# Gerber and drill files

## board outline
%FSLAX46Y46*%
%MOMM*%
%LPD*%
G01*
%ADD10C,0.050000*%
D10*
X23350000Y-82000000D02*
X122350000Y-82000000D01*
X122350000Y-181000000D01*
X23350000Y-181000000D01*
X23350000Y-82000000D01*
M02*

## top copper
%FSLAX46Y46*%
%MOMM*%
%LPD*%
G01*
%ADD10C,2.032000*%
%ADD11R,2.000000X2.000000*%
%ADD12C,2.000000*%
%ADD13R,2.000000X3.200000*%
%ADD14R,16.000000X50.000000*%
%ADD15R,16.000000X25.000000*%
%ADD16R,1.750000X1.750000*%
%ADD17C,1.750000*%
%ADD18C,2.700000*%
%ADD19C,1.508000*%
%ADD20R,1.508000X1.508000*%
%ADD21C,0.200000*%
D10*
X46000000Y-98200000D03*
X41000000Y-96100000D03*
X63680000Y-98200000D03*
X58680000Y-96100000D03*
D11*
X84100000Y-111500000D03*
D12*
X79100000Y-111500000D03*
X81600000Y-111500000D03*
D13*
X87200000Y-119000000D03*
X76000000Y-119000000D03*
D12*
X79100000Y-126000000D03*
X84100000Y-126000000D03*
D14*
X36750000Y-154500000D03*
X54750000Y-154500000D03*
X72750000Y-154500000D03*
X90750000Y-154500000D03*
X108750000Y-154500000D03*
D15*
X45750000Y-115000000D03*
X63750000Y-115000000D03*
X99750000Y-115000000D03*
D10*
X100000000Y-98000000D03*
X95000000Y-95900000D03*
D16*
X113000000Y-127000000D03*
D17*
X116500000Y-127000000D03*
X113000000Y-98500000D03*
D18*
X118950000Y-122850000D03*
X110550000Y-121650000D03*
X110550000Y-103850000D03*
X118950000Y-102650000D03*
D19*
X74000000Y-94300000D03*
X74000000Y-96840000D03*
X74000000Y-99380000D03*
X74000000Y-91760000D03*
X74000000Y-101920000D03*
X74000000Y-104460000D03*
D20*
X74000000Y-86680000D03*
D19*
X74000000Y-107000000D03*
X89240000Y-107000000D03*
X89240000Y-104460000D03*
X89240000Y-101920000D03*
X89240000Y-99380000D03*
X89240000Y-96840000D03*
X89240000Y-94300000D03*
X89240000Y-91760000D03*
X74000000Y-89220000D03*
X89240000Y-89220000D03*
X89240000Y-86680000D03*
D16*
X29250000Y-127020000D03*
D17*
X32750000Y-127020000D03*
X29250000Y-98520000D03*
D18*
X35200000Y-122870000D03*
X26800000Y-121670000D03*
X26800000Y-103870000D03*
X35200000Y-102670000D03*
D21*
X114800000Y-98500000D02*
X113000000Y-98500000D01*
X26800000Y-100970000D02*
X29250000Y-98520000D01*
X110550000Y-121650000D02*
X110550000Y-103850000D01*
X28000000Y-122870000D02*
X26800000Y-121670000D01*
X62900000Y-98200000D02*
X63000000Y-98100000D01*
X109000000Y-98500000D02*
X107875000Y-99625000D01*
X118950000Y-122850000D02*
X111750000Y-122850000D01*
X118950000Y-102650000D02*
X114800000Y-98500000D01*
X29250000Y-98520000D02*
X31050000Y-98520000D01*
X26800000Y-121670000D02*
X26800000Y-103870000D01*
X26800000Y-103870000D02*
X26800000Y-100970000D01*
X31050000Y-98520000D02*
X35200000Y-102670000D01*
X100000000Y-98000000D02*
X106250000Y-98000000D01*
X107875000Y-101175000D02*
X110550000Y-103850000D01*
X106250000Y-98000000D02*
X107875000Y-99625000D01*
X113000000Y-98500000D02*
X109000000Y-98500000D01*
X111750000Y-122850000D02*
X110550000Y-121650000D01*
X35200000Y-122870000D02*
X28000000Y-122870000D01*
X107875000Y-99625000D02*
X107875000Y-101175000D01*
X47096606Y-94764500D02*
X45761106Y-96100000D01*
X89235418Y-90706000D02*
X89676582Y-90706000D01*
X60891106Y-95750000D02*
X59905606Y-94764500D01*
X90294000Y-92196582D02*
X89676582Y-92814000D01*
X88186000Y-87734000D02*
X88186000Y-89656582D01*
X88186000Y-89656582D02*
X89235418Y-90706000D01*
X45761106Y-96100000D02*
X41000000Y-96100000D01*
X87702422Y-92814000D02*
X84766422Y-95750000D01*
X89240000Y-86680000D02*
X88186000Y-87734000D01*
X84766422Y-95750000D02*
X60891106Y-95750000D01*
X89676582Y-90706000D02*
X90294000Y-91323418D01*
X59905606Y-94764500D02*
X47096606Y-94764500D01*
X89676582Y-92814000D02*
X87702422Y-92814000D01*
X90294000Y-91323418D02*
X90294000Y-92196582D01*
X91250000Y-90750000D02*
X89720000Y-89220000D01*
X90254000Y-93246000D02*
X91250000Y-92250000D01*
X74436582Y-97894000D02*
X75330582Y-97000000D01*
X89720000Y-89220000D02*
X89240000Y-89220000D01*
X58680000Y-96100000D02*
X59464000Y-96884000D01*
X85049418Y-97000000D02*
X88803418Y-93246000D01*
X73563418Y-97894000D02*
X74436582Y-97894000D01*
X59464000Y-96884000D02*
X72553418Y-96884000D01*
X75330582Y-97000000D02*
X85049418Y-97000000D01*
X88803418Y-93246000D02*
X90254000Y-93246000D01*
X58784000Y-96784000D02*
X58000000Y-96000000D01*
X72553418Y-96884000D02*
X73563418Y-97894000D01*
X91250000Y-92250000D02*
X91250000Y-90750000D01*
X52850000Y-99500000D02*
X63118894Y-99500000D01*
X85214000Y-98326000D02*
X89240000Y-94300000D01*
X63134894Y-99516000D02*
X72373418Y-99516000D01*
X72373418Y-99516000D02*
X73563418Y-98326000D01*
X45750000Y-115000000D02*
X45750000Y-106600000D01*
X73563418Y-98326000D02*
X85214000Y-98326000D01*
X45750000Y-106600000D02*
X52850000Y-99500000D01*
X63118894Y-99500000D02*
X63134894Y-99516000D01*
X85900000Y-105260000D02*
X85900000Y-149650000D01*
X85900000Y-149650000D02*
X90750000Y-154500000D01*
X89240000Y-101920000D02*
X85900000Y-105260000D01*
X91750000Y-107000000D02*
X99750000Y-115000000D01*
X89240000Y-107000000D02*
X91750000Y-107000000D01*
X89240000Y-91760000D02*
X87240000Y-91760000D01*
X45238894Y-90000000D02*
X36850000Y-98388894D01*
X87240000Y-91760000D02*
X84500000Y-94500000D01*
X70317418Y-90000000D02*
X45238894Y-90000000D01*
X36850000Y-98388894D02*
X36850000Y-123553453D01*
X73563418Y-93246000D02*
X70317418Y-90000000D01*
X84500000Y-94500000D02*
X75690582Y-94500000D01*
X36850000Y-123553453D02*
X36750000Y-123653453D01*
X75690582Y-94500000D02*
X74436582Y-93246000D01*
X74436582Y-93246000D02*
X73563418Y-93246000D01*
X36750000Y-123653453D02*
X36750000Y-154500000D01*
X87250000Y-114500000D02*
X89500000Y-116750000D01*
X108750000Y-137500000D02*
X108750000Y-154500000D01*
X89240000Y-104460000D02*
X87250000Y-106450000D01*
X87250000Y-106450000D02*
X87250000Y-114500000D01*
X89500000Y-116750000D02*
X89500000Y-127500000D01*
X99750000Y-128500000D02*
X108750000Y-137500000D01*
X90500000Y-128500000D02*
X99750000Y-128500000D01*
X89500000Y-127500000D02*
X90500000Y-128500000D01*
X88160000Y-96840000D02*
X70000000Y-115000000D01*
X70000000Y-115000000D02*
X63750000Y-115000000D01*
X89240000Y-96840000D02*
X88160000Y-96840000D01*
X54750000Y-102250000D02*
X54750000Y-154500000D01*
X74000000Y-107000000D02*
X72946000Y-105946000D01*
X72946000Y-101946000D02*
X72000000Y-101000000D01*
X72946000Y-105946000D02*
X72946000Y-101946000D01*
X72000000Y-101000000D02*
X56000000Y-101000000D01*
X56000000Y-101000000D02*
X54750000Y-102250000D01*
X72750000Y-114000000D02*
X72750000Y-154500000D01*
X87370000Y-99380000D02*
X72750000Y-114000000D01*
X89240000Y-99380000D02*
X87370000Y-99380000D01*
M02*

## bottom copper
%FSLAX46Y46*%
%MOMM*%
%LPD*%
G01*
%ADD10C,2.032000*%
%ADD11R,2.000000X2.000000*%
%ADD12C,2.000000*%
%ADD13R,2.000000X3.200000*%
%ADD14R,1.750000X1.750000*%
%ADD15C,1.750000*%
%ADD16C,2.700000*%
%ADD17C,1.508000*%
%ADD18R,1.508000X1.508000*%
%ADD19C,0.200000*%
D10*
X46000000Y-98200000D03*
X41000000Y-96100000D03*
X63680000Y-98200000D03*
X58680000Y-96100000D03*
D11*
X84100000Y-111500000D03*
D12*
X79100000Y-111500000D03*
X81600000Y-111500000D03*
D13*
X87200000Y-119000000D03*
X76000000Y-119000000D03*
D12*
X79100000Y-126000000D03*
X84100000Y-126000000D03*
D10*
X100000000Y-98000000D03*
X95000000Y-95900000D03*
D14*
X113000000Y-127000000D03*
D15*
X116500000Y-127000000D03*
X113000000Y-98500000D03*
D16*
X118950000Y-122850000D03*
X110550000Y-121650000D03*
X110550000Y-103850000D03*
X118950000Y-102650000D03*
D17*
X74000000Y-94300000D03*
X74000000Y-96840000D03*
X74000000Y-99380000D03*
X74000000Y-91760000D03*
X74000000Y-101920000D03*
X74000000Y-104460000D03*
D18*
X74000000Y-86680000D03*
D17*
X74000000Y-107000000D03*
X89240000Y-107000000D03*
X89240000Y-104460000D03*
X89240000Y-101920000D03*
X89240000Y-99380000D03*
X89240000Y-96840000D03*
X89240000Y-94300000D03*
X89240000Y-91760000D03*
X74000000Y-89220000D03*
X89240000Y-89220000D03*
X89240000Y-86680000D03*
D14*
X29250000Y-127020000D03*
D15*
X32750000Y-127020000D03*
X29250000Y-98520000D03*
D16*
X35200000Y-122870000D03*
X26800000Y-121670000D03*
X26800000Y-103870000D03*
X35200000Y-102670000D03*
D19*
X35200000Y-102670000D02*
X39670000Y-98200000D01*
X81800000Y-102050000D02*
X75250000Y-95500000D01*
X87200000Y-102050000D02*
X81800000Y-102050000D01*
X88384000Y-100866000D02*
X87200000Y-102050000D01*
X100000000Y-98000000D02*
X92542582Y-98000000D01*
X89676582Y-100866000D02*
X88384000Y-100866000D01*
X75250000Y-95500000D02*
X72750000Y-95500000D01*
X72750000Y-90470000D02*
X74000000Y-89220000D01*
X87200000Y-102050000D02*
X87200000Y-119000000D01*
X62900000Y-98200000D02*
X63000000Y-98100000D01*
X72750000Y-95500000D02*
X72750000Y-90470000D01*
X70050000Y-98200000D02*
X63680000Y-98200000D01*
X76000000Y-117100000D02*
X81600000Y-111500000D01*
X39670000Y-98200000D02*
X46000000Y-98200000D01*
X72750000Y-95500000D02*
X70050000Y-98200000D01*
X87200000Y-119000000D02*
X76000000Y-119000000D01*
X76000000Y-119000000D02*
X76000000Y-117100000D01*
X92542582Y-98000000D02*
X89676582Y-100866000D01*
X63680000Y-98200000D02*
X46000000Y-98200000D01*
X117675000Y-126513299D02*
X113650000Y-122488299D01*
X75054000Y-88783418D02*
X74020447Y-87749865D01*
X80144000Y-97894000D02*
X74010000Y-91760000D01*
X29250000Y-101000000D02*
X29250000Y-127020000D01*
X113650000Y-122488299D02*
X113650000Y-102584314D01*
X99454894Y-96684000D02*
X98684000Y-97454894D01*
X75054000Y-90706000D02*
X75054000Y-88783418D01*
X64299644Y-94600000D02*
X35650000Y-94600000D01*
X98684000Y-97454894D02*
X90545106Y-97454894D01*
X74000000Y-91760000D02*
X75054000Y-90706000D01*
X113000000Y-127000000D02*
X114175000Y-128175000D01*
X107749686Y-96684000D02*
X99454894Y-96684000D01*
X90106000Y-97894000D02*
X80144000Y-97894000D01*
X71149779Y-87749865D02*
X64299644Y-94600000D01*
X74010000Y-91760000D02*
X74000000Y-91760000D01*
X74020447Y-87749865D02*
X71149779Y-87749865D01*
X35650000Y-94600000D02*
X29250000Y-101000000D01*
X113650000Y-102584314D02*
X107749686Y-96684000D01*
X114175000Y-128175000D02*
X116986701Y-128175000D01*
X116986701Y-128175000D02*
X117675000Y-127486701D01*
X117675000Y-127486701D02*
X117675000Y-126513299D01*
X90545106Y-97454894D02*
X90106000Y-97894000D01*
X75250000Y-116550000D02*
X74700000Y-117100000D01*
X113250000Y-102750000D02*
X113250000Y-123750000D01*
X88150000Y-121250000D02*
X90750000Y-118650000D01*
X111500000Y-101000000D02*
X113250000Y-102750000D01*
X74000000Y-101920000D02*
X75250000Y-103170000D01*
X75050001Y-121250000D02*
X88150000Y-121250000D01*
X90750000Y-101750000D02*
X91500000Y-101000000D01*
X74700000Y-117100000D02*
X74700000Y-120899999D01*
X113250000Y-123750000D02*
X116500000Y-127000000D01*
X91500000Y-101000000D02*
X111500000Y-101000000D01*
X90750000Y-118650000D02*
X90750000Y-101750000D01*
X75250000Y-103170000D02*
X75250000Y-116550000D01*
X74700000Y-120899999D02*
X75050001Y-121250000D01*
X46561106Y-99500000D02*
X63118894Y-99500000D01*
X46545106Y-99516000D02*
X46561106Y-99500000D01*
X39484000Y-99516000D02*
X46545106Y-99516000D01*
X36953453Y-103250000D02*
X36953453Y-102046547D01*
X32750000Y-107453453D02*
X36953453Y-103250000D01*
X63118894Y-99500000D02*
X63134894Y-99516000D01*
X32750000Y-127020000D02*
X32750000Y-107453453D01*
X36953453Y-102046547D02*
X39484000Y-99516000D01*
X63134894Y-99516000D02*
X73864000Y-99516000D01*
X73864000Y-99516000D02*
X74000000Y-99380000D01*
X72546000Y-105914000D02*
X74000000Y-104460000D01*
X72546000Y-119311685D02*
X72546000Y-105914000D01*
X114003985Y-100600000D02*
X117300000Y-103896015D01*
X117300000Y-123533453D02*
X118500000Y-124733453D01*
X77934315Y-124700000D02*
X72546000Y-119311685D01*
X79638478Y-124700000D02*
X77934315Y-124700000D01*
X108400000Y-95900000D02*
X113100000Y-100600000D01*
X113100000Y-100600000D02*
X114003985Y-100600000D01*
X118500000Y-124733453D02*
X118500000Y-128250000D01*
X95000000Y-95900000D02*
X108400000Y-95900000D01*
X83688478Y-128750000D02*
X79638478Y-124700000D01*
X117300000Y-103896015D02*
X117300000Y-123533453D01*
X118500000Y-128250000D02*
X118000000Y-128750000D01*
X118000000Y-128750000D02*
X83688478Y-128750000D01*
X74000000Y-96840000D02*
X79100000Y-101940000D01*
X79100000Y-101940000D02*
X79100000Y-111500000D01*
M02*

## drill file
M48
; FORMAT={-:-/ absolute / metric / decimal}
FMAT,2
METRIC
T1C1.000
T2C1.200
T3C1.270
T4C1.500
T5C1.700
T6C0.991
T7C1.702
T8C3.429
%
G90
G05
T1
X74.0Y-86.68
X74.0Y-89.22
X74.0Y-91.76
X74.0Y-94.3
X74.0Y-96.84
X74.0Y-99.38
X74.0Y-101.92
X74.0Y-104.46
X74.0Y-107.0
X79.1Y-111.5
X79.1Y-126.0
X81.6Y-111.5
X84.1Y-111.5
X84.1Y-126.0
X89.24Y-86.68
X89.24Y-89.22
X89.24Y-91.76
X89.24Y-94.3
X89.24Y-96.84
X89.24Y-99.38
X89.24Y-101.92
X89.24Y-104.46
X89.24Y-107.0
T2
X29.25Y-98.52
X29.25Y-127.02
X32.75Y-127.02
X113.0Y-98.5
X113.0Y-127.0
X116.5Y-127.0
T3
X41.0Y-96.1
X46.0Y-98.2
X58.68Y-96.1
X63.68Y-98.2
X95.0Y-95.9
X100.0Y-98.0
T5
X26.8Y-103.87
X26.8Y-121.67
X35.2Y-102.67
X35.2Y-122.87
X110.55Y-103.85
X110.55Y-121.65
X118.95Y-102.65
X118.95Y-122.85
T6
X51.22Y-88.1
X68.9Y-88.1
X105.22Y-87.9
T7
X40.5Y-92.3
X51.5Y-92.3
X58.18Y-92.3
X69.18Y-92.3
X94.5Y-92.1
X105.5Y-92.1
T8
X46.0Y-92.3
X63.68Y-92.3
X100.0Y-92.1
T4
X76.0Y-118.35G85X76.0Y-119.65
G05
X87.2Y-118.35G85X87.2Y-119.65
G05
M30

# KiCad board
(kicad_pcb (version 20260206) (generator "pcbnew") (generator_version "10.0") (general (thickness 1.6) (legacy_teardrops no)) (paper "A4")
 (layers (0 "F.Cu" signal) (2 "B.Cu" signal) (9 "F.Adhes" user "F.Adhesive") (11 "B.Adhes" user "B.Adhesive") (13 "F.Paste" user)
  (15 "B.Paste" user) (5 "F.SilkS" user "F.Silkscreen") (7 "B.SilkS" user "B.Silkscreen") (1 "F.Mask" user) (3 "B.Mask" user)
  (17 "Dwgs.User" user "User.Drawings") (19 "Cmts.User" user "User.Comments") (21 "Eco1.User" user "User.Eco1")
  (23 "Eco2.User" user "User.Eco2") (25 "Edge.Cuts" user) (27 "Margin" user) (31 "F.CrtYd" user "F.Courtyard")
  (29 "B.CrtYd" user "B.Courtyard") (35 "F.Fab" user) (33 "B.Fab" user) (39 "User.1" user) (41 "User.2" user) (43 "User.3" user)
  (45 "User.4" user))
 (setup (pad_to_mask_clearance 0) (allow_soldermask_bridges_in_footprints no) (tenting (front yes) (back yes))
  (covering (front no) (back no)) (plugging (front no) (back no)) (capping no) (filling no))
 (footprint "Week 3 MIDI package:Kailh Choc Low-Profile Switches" (layer "F.Cu") (at 46 92.3)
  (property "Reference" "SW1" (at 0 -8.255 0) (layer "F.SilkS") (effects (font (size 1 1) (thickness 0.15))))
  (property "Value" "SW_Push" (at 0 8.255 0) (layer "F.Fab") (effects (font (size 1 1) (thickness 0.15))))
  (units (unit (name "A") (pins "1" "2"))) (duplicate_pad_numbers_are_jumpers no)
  (pad "" np_thru_hole circle (at -5.5 0) (size 1.7018 1.7018) (drill 1.7018) (layers "*.Cu" "*.Mask"))
  (pad "" np_thru_hole circle (at 0 0) (size 3.429 3.429) (drill 3.429) (layers "*.Cu" "*.Mask"))
  (pad "" np_thru_hole circle (at 5.22 -4.2) (size 0.9906 0.9906) (drill 0.9906) (layers "*.Cu" "*.Mask"))
  (pad "" np_thru_hole circle (at 5.5 0) (size 1.7018 1.7018) (drill 1.7018) (layers "*.Cu" "*.Mask"))
  (pad "1" thru_hole circle (at 0 5.9) (size 2.032 2.032) (drill 1.27) (layers "*.Cu" "*.Mask") (remove_unused_layers no) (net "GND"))
  (pad "2" thru_hole circle (at -5 3.8) (size 2.032 2.032) (drill 1.27) (layers "*.Cu" "*.Mask") (remove_unused_layers no) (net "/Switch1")))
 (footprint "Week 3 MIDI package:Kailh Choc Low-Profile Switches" (layer "F.Cu") (at 63.68 92.3)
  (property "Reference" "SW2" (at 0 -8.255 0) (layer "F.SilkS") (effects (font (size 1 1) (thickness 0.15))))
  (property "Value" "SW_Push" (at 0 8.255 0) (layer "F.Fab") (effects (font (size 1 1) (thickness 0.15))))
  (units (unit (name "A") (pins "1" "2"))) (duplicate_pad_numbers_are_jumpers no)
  (pad "" np_thru_hole circle (at -5.5 0) (size 1.7018 1.7018) (drill 1.7018) (layers "*.Cu" "*.Mask"))
  (pad "" np_thru_hole circle (at 0 0) (size 3.429 3.429) (drill 3.429) (layers "*.Cu" "*.Mask"))
  (pad "" np_thru_hole circle (at 5.22 -4.2) (size 0.9906 0.9906) (drill 0.9906) (layers "*.Cu" "*.Mask"))
  (pad "" np_thru_hole circle (at 5.5 0) (size 1.7018 1.7018) (drill 1.7018) (layers "*.Cu" "*.Mask"))
  (pad "1" thru_hole circle (at 0 5.9) (size 2.032 2.032) (drill 1.27) (layers "*.Cu" "*.Mask") (remove_unused_layers no) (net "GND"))
  (pad "2" thru_hole circle (at -5 3.8) (size 2.032 2.032) (drill 1.27) (layers "*.Cu" "*.Mask") (remove_unused_layers no) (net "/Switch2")))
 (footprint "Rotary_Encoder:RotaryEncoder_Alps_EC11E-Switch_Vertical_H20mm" (layer "F.Cu") (at 84.1 111.5 -90)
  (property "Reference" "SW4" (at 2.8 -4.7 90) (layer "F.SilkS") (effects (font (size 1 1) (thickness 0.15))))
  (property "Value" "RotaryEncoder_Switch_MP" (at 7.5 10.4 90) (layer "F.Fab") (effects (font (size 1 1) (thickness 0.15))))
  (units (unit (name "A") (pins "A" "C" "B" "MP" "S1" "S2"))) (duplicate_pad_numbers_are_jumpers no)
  (pad "A" thru_hole rect (at 0 0 270) (size 2 2) (drill 1) (layers "*.Cu" "*.Mask") (remove_unused_layers no) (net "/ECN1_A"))
  (pad "B" thru_hole circle (at 0 5 270) (size 2 2) (drill 1) (layers "*.Cu" "*.Mask") (remove_unused_layers no) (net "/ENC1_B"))
  (pad "C" thru_hole circle (at 0 2.5 270) (size 2 2) (drill 1) (layers "*.Cu" "*.Mask") (remove_unused_layers no) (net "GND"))
  (pad "MP" thru_hole rect (at 7.5 -3.1 270) (size 3.2 2) (drill oval 2.8 1.5) (layers "*.Cu" "*.Mask") (remove_unused_layers no)
   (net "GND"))
  (pad "MP" thru_hole rect (at 7.5 8.1 270) (size 3.2 2) (drill oval 2.8 1.5) (layers "*.Cu" "*.Mask") (remove_unused_layers no) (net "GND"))
  (pad "S1" thru_hole circle (at 14.5 5 270) (size 2 2) (drill 1) (layers "*.Cu" "*.Mask") (remove_unused_layers no)
   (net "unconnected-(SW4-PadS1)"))
  (pad "S2" thru_hole circle (at 14.5 0 270) (size 2 2) (drill 1) (layers "*.Cu" "*.Mask") (remove_unused_layers no)
   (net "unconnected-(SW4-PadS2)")))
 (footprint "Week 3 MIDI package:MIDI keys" (layer "F.Cu") (at 28.75 179.5)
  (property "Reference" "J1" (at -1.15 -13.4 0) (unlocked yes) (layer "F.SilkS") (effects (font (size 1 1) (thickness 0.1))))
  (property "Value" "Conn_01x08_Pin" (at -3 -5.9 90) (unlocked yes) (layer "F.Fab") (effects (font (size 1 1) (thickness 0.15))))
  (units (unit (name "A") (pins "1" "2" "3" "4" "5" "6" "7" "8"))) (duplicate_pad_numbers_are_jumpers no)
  (pad "1" smd rect (at 8 -25) (size 16 50) (layers "F.Cu" "F.Mask") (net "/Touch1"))
  (pad "2" smd rect (at 26 -25) (size 16 50) (layers "F.Cu" "F.Mask") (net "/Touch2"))
  (pad "3" smd rect (at 44 -25) (size 16 50) (layers "F.Cu" "F.Mask") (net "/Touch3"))
  (pad "4" smd rect (at 62 -25) (size 16 50) (layers "F.Cu" "F.Mask") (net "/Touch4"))
  (pad "5" smd rect (at 80 -25) (size 16 50) (layers "F.Cu" "F.Mask") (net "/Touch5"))
  (pad "6" smd rect (at 17 -64.5) (size 16 25) (layers "F.Cu" "F.Mask") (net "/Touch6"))
  (pad "7" smd rect (at 35 -64.5) (size 16 25) (layers "F.Cu" "F.Mask") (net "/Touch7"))
  (pad "8" smd rect (at 71 -64.5) (size 16 25) (layers "F.Cu" "F.Mask") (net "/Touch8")))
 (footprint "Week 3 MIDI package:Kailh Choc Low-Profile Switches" (layer "F.Cu") (at 100 92.1)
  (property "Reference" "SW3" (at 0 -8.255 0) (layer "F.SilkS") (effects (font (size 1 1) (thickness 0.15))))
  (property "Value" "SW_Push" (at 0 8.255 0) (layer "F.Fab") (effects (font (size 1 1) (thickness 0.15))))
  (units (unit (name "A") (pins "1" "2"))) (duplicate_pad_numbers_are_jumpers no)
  (pad "" np_thru_hole circle (at -5.5 0) (size 1.7018 1.7018) (drill 1.7018) (layers "*.Cu" "*.Mask"))
  (pad "" np_thru_hole circle (at 0 0) (size 3.429 3.429) (drill 3.429) (layers "*.Cu" "*.Mask"))
  (pad "" np_thru_hole circle (at 5.22 -4.2) (size 0.9906 0.9906) (drill 0.9906) (layers "*.Cu" "*.Mask"))
  (pad "" np_thru_hole circle (at 5.5 0) (size 1.7018 1.7018) (drill 1.7018) (layers "*.Cu" "*.Mask"))
  (pad "1" thru_hole circle (at 0 5.9) (size 2.032 2.032) (drill 1.27) (layers "*.Cu" "*.Mask") (remove_unused_layers no) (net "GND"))
  (pad "2" thru_hole circle (at -5 3.8) (size 2.032 2.032) (drill 1.27) (layers "*.Cu" "*.Mask") (remove_unused_layers no) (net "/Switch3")))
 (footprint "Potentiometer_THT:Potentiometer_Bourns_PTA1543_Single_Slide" (layer "F.Cu") (at 113 127 90)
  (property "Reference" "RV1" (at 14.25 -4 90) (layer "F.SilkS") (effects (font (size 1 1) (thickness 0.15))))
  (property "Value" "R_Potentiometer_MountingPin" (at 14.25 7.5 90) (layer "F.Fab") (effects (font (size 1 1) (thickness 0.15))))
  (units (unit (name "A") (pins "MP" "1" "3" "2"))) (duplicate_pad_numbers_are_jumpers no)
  (pad "1" thru_hole rect (at 0 0 90) (size 1.75 1.75) (drill 1.2) (layers "*.Cu" "*.Mask") (remove_unused_layers no) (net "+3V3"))
  (pad "2" thru_hole circle (at 0 3.5 90) (size 1.75 1.75) (drill 1.2) (layers "*.Cu" "*.Mask") (remove_unused_layers no) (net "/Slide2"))
  (pad "3" thru_hole circle (at 28.5 0 90) (size 1.75 1.75) (drill 1.2) (layers "*.Cu" "*.Mask") (remove_unused_layers no) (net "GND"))
  (pad "MP" thru_hole circle (at 4.15 5.95 90) (size 2.7 2.7) (drill 1.7) (layers "*.Cu" "*.Mask") (remove_unused_layers no) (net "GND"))
  (pad "MP" thru_hole circle (at 5.35 -2.45 90) (size 2.7 2.7) (drill 1.7) (layers "*.Cu" "*.Mask") (remove_unused_layers no) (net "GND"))
  (pad "MP" thru_hole circle (at 23.15 -2.45 90) (size 2.7 2.7) (drill 1.7) (layers "*.Cu" "*.Mask") (remove_unused_layers no) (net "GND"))
  (pad "MP" thru_hole circle (at 24.35 5.95 90) (size 2.7 2.7) (drill 1.7) (layers "*.Cu" "*.Mask") (remove_unused_layers no) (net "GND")))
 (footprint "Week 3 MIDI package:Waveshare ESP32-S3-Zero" (layer "F.Cu") (at 81.62 96.84)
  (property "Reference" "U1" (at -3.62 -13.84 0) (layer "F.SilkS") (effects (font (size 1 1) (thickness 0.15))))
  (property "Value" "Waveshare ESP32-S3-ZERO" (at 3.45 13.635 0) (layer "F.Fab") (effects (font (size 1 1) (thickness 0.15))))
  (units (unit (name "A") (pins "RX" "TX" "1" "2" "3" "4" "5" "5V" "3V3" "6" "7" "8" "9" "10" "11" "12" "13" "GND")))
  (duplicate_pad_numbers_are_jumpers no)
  (pad "1" thru_hole circle (at -7.62 -2.54) (size 1.508 1.508) (drill 1) (layers "*.Cu" "*.Mask") (remove_unused_layers no) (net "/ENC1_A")
   (solder_mask_margin 0.102))
  (pad "2" thru_hole circle (at -7.62 0) (size 1.508 1.508) (drill 1) (layers "*.Cu" "*.Mask") (remove_unused_layers no) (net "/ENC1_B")
   (solder_mask_margin 0.102))
  (pad "3" thru_hole circle (at -7.62 2.54) (size 1.508 1.508) (drill 1) (layers "*.Cu" "*.Mask") (remove_unused_layers no) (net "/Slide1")
   (solder_mask_margin 0.102))
  (pad "3V3" thru_hole circle (at -7.62 -5.08) (size 1.508 1.508) (drill 1) (layers "*.Cu" "*.Mask") (remove_unused_layers no) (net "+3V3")
   (solder_mask_margin 0.102))
  (pad "4" thru_hole circle (at -7.62 5.08) (size 1.508 1.508) (drill 1) (layers "*.Cu" "*.Mask") (remove_unused_layers no) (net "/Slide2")
   (solder_mask_margin 0.102))
  (pad "5" thru_hole circle (at -7.62 7.62) (size 1.508 1.508) (drill 1) (layers "*.Cu" "*.Mask") (remove_unused_layers no) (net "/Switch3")
   (solder_mask_margin 0.102))
  (pad "5V" thru_hole rect (at -7.62 -10.16) (size 1.508 1.508) (drill 1) (layers "*.Cu" "*.Mask") (remove_unused_layers no) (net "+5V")
   (solder_mask_margin 0.102))
  (pad "6" thru_hole circle (at -7.62 10.16) (size 1.508 1.508) (drill 1) (layers "*.Cu" "*.Mask") (remove_unused_layers no) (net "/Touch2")
   (solder_mask_margin 0.102))
  (pad "7" thru_hole circle (at 7.62 10.16) (size 1.508 1.508) (drill 1) (layers "*.Cu" "*.Mask") (remove_unused_layers no) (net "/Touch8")
   (solder_mask_margin 0.102))
  (pad "8" thru_hole circle (at 7.62 7.62) (size 1.508 1.508) (drill 1) (layers "*.Cu" "*.Mask") (remove_unused_layers no) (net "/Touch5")
   (solder_mask_margin 0.102))
  (pad "9" thru_hole circle (at 7.62 5.08) (size 1.508 1.508) (drill 1) (layers "*.Cu" "*.Mask") (remove_unused_layers no) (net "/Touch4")
   (solder_mask_margin 0.102))
  (pad "10" thru_hole circle (at 7.62 2.54) (size 1.508 1.508) (drill 1) (layers "*.Cu" "*.Mask") (remove_unused_layers no) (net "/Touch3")
   (solder_mask_margin 0.102))
  (pad "11" thru_hole circle (at 7.62 0) (size 1.508 1.508) (drill 1) (layers "*.Cu" "*.Mask") (remove_unused_layers no) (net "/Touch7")
   (solder_mask_margin 0.102))
  (pad "12" thru_hole circle (at 7.62 -2.54) (size 1.508 1.508) (drill 1) (layers "*.Cu" "*.Mask") (remove_unused_layers no) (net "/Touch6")
   (solder_mask_margin 0.102))
  (pad "13" thru_hole circle (at 7.62 -5.08) (size 1.508 1.508) (drill 1) (layers "*.Cu" "*.Mask") (remove_unused_layers no) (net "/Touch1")
   (solder_mask_margin 0.102))
  (pad "GND" thru_hole circle (at -7.62 -7.62) (size 1.508 1.508) (drill 1) (layers "*.Cu" "*.Mask") (remove_unused_layers no) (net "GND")
   (solder_mask_margin 0.102))
  (pad "RX" thru_hole circle (at 7.62 -7.62) (size 1.508 1.508) (drill 1) (layers "*.Cu" "*.Mask") (remove_unused_layers no)
   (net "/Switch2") (solder_mask_margin 0.102))
  (pad "TX" thru_hole circle (at 7.62 -10.16) (size 1.508 1.508) (drill 1) (layers "*.Cu" "*.Mask") (remove_unused_layers no)
   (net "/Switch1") (solder_mask_margin 0.102)))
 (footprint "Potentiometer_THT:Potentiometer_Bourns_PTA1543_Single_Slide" (layer "F.Cu") (at 29.25 127.02 90)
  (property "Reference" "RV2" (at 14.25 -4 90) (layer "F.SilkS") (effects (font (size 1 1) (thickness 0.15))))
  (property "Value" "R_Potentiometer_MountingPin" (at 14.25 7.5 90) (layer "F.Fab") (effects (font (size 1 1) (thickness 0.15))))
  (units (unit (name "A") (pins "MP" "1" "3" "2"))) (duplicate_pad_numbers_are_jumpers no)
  (pad "1" thru_hole rect (at 0 0 90) (size 1.75 1.75) (drill 1.2) (layers "*.Cu" "*.Mask") (remove_unused_layers no) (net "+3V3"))
  (pad "2" thru_hole circle (at 0 3.5 90) (size 1.75 1.75) (drill 1.2) (layers "*.Cu" "*.Mask") (remove_unused_layers no) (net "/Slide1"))
  (pad "3" thru_hole circle (at 28.5 0 90) (size 1.75 1.75) (drill 1.2) (layers "*.Cu" "*.Mask") (remove_unused_layers no) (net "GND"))
  (pad "MP" thru_hole circle (at 4.15 5.95 90) (size 2.7 2.7) (drill 1.7) (layers "*.Cu" "*.Mask") (remove_unused_layers no) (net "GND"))
  (pad "MP" thru_hole circle (at 5.35 -2.45 90) (size 2.7 2.7) (drill 1.7) (layers "*.Cu" "*.Mask") (remove_unused_layers no) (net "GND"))
  (pad "MP" thru_hole circle (at 23.15 -2.45 90) (size 2.7 2.7) (drill 1.7) (layers "*.Cu" "*.Mask") (remove_unused_layers no) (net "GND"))
  (pad "MP" thru_hole circle (at 24.35 5.95 90) (size 2.7 2.7) (drill 1.7) (layers "*.Cu" "*.Mask") (remove_unused_layers no) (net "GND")))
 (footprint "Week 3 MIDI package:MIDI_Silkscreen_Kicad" (layer "B.Cu") (at 76.35 171.65 180)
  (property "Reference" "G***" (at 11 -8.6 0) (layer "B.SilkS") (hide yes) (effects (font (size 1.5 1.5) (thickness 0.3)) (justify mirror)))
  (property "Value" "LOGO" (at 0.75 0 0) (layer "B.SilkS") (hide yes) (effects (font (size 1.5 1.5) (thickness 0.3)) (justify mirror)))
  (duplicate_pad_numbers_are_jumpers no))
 (gr_rect (start 23.35 82) (end 122.35 181) (stroke (width 0.05) (type default)) (fill no) (layer "Edge.Cuts"))
 (segment (start 114.8 98.5) (end 113 98.5) (width 0.2) (layer "F.Cu") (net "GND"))
 (segment (start 26.8 100.97) (end 29.25 98.52) (width 0.2) (layer "F.Cu") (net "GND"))
 (segment (start 110.55 121.65) (end 110.55 103.85) (width 0.2) (layer "F.Cu") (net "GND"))
 (segment (start 28 122.87) (end 26.8 121.67) (width 0.2) (layer "F.Cu") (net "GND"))
 (segment (start 62.9 98.2) (end 63 98.1) (width 0.2) (layer "F.Cu") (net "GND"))
 (segment (start 109 98.5) (end 107.875 99.625) (width 0.2) (layer "F.Cu") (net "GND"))
 (segment (start 118.95 122.85) (end 111.75 122.85) (width 0.2) (layer "F.Cu") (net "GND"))
 (segment (start 118.95 102.65) (end 114.8 98.5) (width 0.2) (layer "F.Cu") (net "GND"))
 (segment (start 29.25 98.52) (end 31.05 98.52) (width 0.2) (layer "F.Cu") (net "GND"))
 (segment (start 26.8 121.67) (end 26.8 103.87) (width 0.2) (layer "F.Cu") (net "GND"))
 (segment (start 26.8 103.87) (end 26.8 100.97) (width 0.2) (layer "F.Cu") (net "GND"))
 (segment (start 31.05 98.52) (end 35.2 102.67) (width 0.2) (layer "F.Cu") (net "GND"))
 (segment (start 100 98) (end 106.25 98) (width 0.2) (layer "F.Cu") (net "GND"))
 (segment (start 107.875 101.175) (end 110.55 103.85) (width 0.2) (layer "F.Cu") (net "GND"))
 (segment (start 106.25 98) (end 107.875 99.625) (width 0.2) (layer "F.Cu") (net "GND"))
 (segment (start 113 98.5) (end 109 98.5) (width 0.2) (layer "F.Cu") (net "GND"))
 (segment (start 111.75 122.85) (end 110.55 121.65) (width 0.2) (layer "F.Cu") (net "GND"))
 (segment (start 35.2 122.87) (end 28 122.87) (width 0.2) (layer "F.Cu") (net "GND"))
 (segment (start 107.875 99.625) (end 107.875 101.175) (width 0.2) (layer "F.Cu") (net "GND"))
 (segment (start 35.2 102.67) (end 39.67 98.2) (width 0.2) (layer "B.Cu") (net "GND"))
 (segment (start 81.8 102.05) (end 75.25 95.5) (width 0.2) (layer "B.Cu") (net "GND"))
 (segment (start 87.2 102.05) (end 81.8 102.05) (width 0.2) (layer "B.Cu") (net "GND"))
 (segment (start 88.384 100.866) (end 87.2 102.05) (width 0.2) (layer "B.Cu") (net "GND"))
 (segment (start 100 98) (end 92.542582 98) (width 0.2) (layer "B.Cu") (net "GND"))
 (segment (start 89.676582 100.866) (end 88.384 100.866) (width 0.2) (layer "B.Cu") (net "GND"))
 (segment (start 75.25 95.5) (end 72.75 95.5) (width 0.2) (layer "B.Cu") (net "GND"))
 (segment (start 72.75 90.47) (end 74 89.22) (width 0.2) (layer "B.Cu") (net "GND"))
 (segment (start 87.2 102.05) (end 87.2 119) (width 0.2) (layer "B.Cu") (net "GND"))
 (segment (start 62.9 98.2) (end 63 98.1) (width 0.2) (layer "B.Cu") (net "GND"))
 (segment (start 72.75 95.5) (end 72.75 90.47) (width 0.2) (layer "B.Cu") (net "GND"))
 (segment (start 70.05 98.2) (end 63.68 98.2) (width 0.2) (layer "B.Cu") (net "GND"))
 (segment (start 76 117.1) (end 81.6 111.5) (width 0.2) (layer "B.Cu") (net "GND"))
 (segment (start 39.67 98.2) (end 46 98.2) (width 0.2) (layer "B.Cu") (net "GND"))
 (segment (start 72.75 95.5) (end 70.05 98.2) (width 0.2) (layer "B.Cu") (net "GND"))
 (segment (start 87.2 119) (end 76 119) (width 0.2) (layer "B.Cu") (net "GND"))
 (segment (start 76 119) (end 76 117.1) (width 0.2) (layer "B.Cu") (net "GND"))
 (segment (start 92.542582 98) (end 89.676582 100.866) (width 0.2) (layer "B.Cu") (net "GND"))
 (segment (start 63.68 98.2) (end 46 98.2) (width 0.2) (layer "B.Cu") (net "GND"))
 (segment (start 117.675 126.513299) (end 113.65 122.488299) (width 0.2) (layer "B.Cu") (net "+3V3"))
 (segment (start 75.054 88.783418) (end 74.020447 87.749865) (width 0.2) (layer "B.Cu") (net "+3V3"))
 (segment (start 80.144 97.894) (end 74.01 91.76) (width 0.2) (layer "B.Cu") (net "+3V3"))
 (segment (start 29.25 101) (end 29.25 127.02) (width 0.2) (layer "B.Cu") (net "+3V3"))
 (segment (start 113.65 122.488299) (end 113.65 102.584314) (width 0.2) (layer "B.Cu") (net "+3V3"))
 (segment (start 99.454894 96.684) (end 98.684 97.454894) (width 0.2) (layer "B.Cu") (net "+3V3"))
 (segment (start 75.054 90.706) (end 75.054 88.783418) (width 0.2) (layer "B.Cu") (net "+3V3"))
 (segment (start 64.299644 94.6) (end 35.65 94.6) (width 0.2) (layer "B.Cu") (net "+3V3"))
 (segment (start 98.684 97.454894) (end 90.545106 97.454894) (width 0.2) (layer "B.Cu") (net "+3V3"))
 (segment (start 74 91.76) (end 75.054 90.706) (width 0.2) (layer "B.Cu") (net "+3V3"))
 (segment (start 113 127) (end 114.175 128.175) (width 0.2) (layer "B.Cu") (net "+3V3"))
 (segment (start 107.749686 96.684) (end 99.454894 96.684) (width 0.2) (layer "B.Cu") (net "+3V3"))
 (segment (start 90.106 97.894) (end 80.144 97.894) (width 0.2) (layer "B.Cu") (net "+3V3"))
 (segment (start 71.149779 87.749865) (end 64.299644 94.6) (width 0.2) (layer "B.Cu") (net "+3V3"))
 (segment (start 74.01 91.76) (end 74 91.76) (width 0.2) (layer "B.Cu") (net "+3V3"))
 (segment (start 74.020447 87.749865) (end 71.149779 87.749865) (width 0.2) (layer "B.Cu") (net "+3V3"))
 (segment (start 35.65 94.6) (end 29.25 101) (width 0.2) (layer "B.Cu") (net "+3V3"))
 (segment (start 113.65 102.584314) (end 107.749686 96.684) (width 0.2) (layer "B.Cu") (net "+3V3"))
 (segment (start 114.175 128.175) (end 116.986701 128.175) (width 0.2) (layer "B.Cu") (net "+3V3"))
 (segment (start 116.986701 128.175) (end 117.675 127.486701) (width 0.2) (layer "B.Cu") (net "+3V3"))
 (segment (start 117.675 127.486701) (end 117.675 126.513299) (width 0.2) (layer "B.Cu") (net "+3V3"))
 (segment (start 90.545106 97.454894) (end 90.106 97.894) (width 0.2) (layer "B.Cu") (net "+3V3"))
 (segment (start 75.25 116.55) (end 74.7 117.1) (width 0.2) (layer "B.Cu") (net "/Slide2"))
 (segment (start 113.25 102.75) (end 113.25 123.75) (width 0.2) (layer "B.Cu") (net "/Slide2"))
 (segment (start 88.15 121.25) (end 90.75 118.65) (width 0.2) (layer "B.Cu") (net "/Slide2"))
 (segment (start 111.5 101) (end 113.25 102.75) (width 0.2) (layer "B.Cu") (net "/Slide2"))
 (segment (start 74 101.92) (end 75.25 103.17) (width 0.2) (layer "B.Cu") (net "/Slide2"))
 (segment (start 75.050001 121.25) (end 88.15 121.25) (width 0.2) (layer "B.Cu") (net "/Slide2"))
 (segment (start 90.75 101.75) (end 91.5 101) (width 0.2) (layer "B.Cu") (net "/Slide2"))
 (segment (start 74.7 117.1) (end 74.7 120.899999) (width 0.2) (layer "B.Cu") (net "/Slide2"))
 (segment (start 113.25 123.75) (end 116.5 127) (width 0.2) (layer "B.Cu") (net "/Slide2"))
 (segment (start 91.5 101) (end 111.5 101) (width 0.2) (layer "B.Cu") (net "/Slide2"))
 (segment (start 90.75 118.65) (end 90.75 101.75) (width 0.2) (layer "B.Cu") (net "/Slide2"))
 (segment (start 75.25 103.17) (end 75.25 116.55) (width 0.2) (layer "B.Cu") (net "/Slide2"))
 (segment (start 74.7 120.899999) (end 75.050001 121.25) (width 0.2) (layer "B.Cu") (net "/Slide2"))
 (segment (start 46.561106 99.5) (end 63.118894 99.5) (width 0.2) (layer "B.Cu") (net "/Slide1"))
 (segment (start 46.545106 99.516) (end 46.561106 99.5) (width 0.2) (layer "B.Cu") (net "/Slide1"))
 (segment (start 39.484 99.516) (end 46.545106 99.516) (width 0.2) (layer "B.Cu") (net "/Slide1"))
 (segment (start 36.953453 103.25) (end 36.953453 102.046547) (width 0.2) (layer "B.Cu") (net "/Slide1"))
 (segment (start 32.75 107.453453) (end 36.953453 103.25) (width 0.2) (layer "B.Cu") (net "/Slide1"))
 (segment (start 63.118894 99.5) (end 63.134894 99.516) (width 0.2) (layer "B.Cu") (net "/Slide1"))
 (segment (start 32.75 127.02) (end 32.75 107.453453) (width 0.2) (layer "B.Cu") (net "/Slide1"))
 (segment (start 36.953453 102.046547) (end 39.484 99.516) (width 0.2) (layer "B.Cu") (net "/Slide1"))
 (segment (start 63.134894 99.516) (end 73.864 99.516) (width 0.2) (layer "B.Cu") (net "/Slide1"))
 (segment (start 73.864 99.516) (end 74 99.38) (width 0.2) (layer "B.Cu") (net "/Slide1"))
 (segment (start 47.096606 94.7645) (end 45.761106 96.1) (width 0.2) (layer "F.Cu") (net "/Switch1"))
 (segment (start 89.235418 90.706) (end 89.676582 90.706) (width 0.2) (layer "F.Cu") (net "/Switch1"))
 (segment (start 60.891106 95.75) (end 59.905606 94.7645) (width 0.2) (layer "F.Cu") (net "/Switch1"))
 (segment (start 90.294 92.196582) (end 89.676582 92.814) (width 0.2) (layer "F.Cu") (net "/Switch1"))
 (segment (start 88.186 87.734) (end 88.186 89.656582) (width 0.2) (layer "F.Cu") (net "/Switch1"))
 (segment (start 88.186 89.656582) (end 89.235418 90.706) (width 0.2) (layer "F.Cu") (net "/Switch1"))
 (segment (start 45.761106 96.1) (end 41 96.1) (width 0.2) (layer "F.Cu") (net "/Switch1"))
 (segment (start 87.702422 92.814) (end 84.766422 95.75) (width 0.2) (layer "F.Cu") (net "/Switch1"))
 (segment (start 89.24 86.68) (end 88.186 87.734) (width 0.2) (layer "F.Cu") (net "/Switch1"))
 (segment (start 84.766422 95.75) (end 60.891106 95.75) (width 0.2) (layer "F.Cu") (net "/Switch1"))
 (segment (start 89.676582 90.706) (end 90.294 91.323418) (width 0.2) (layer "F.Cu") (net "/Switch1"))
 (segment (start 59.905606 94.7645) (end 47.096606 94.7645) (width 0.2) (layer "F.Cu") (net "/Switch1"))
 (segment (start 89.676582 92.814) (end 87.702422 92.814) (width 0.2) (layer "F.Cu") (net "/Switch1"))
 (segment (start 90.294 91.323418) (end 90.294 92.196582) (width 0.2) (layer "F.Cu") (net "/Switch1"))
 (segment (start 91.25 90.75) (end 89.72 89.22) (width 0.2) (layer "F.Cu") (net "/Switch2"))
 (segment (start 90.254 93.246) (end 91.25 92.25) (width 0.2) (layer "F.Cu") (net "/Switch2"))
 (segment (start 74.436582 97.894) (end 75.330582 97) (width 0.2) (layer "F.Cu") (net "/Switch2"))
 (segment (start 89.72 89.22) (end 89.24 89.22) (width 0.2) (layer "F.Cu") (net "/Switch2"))
 (segment (start 58.68 96.1) (end 59.464 96.884) (width 0.2) (layer "F.Cu") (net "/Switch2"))
 (segment (start 85.049418 97) (end 88.803418 93.246) (width 0.2) (layer "F.Cu") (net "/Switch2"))
 (segment (start 73.563418 97.894) (end 74.436582 97.894) (width 0.2) (layer "F.Cu") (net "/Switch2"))
 (segment (start 59.464 96.884) (end 72.553418 96.884) (width 0.2) (layer "F.Cu") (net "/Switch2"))
 (segment (start 75.330582 97) (end 85.049418 97) (width 0.2) (layer "F.Cu") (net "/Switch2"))
 (segment (start 88.803418 93.246) (end 90.254 93.246) (width 0.2) (layer "F.Cu") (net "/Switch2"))
 (segment (start 58.784 96.784) (end 58 96) (width 0.2) (layer "F.Cu") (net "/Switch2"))
 (segment (start 72.553418 96.884) (end 73.563418 97.894) (width 0.2) (layer "F.Cu") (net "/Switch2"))
 (segment (start 91.25 92.25) (end 91.25 90.75) (width 0.2) (layer "F.Cu") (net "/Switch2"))
 (segment (start 72.546 105.914) (end 74 104.46) (width 0.2) (layer "B.Cu") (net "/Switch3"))
 (segment (start 72.546 119.311685) (end 72.546 105.914) (width 0.2) (layer "B.Cu") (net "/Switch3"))
 (segment (start 114.003985 100.6) (end 117.3 103.896015) (width 0.2) (layer "B.Cu") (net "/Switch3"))
 (segment (start 117.3 123.533453) (end 118.5 124.733453) (width 0.2) (layer "B.Cu") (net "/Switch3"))
 (segment (start 77.934315 124.7) (end 72.546 119.311685) (width 0.2) (layer "B.Cu") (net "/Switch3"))
 (segment (start 79.638478 124.7) (end 77.934315 124.7) (width 0.2) (layer "B.Cu") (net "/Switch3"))
 (segment (start 108.4 95.9) (end 113.1 100.6) (width 0.2) (layer "B.Cu") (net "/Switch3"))
 (segment (start 113.1 100.6) (end 114.003985 100.6) (width 0.2) (layer "B.Cu") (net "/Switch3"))
 (segment (start 118.5 124.733453) (end 118.5 128.25) (width 0.2) (layer "B.Cu") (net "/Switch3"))
 (segment (start 95 95.9) (end 108.4 95.9) (width 0.2) (layer "B.Cu") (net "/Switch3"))
 (segment (start 83.688478 128.75) (end 79.638478 124.7) (width 0.2) (layer "B.Cu") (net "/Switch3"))
 (segment (start 117.3 103.896015) (end 117.3 123.533453) (width 0.2) (layer "B.Cu") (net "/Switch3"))
 (segment (start 118.5 128.25) (end 118 128.75) (width 0.2) (layer "B.Cu") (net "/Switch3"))
 (segment (start 118 128.75) (end 83.688478 128.75) (width 0.2) (layer "B.Cu") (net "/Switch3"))
 (segment (start 74 96.84) (end 79.1 101.94) (width 0.2) (layer "B.Cu") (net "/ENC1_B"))
 (segment (start 79.1 101.94) (end 79.1 111.5) (width 0.2) (layer "B.Cu") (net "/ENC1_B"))
 (segment (start 52.85 99.5) (end 63.118894 99.5) (width 0.2) (layer "F.Cu") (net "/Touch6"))
 (segment (start 85.214 98.326) (end 89.24 94.3) (width 0.2) (layer "F.Cu") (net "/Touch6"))
 (segment (start 63.134894 99.516) (end 72.373418 99.516) (width 0.2) (layer "F.Cu") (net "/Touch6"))
 (segment (start 72.373418 99.516) (end 73.563418 98.326) (width 0.2) (layer "F.Cu") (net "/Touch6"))
 (segment (start 45.75 115) (end 45.75 106.6) (width 0.2) (layer "F.Cu") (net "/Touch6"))
 (segment (start 73.563418 98.326) (end 85.214 98.326) (width 0.2) (layer "F.Cu") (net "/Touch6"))
 (segment (start 45.75 106.6) (end 52.85 99.5) (width 0.2) (layer "F.Cu") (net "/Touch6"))
 (segment (start 63.118894 99.5) (end 63.134894 99.516) (width 0.2) (layer "F.Cu") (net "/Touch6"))
 (segment (start 85.9 105.26) (end 85.9 149.65) (width 0.2) (layer "F.Cu") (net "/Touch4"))
 (segment (start 85.9 149.65) (end 90.75 154.5) (width 0.2) (layer "F.Cu") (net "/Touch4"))
 (segment (start 89.24 101.92) (end 85.9 105.26) (width 0.2) (layer "F.Cu") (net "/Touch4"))
 (segment (start 91.75 107) (end 99.75 115) (width 0.2) (layer "F.Cu") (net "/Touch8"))
 (segment (start 89.24 107) (end 91.75 107) (width 0.2) (layer "F.Cu") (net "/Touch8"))
 (segment (start 89.24 91.76) (end 87.24 91.76) (width 0.2) (layer "F.Cu") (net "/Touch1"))
 (segment (start 45.238894 90) (end 36.85 98.388894) (width 0.2) (layer "F.Cu") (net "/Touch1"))
 (segment (start 87.24 91.76) (end 84.5 94.5) (width 0.2) (layer "F.Cu") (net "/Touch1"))
 (segment (start 70.317418 90) (end 45.238894 90) (width 0.2) (layer "F.Cu") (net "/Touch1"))
 (segment (start 36.85 98.388894) (end 36.85 123.553453) (width 0.2) (layer "F.Cu") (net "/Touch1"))
 (segment (start 73.563418 93.246) (end 70.317418 90) (width 0.2) (layer "F.Cu") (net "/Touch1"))
 (segment (start 84.5 94.5) (end 75.690582 94.5) (width 0.2) (layer "F.Cu") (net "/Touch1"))
 (segment (start 36.85 123.553453) (end 36.75 123.653453) (width 0.2) (layer "F.Cu") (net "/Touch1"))
 (segment (start 75.690582 94.5) (end 74.436582 93.246) (width 0.2) (layer "F.Cu") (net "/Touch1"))
 (segment (start 74.436582 93.246) (end 73.563418 93.246) (width 0.2) (layer "F.Cu") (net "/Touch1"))
 (segment (start 36.75 123.653453) (end 36.75 154.5) (width 0.2) (layer "F.Cu") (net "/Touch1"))
 (segment (start 87.25 114.5) (end 89.5 116.75) (width 0.2) (layer "F.Cu") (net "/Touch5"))
 (segment (start 108.75 137.5) (end 108.75 154.5) (width 0.2) (layer "F.Cu") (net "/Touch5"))
 (segment (start 89.24 104.46) (end 87.25 106.45) (width 0.2) (layer "F.Cu") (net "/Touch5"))
 (segment (start 87.25 106.45) (end 87.25 114.5) (width 0.2) (layer "F.Cu") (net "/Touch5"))
 (segment (start 89.5 116.75) (end 89.5 127.5) (width 0.2) (layer "F.Cu") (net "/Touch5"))
 (segment (start 99.75 128.5) (end 108.75 137.5) (width 0.2) (layer "F.Cu") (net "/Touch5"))
 (segment (start 90.5 128.5) (end 99.75 128.5) (width 0.2) (layer "F.Cu") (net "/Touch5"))
 (segment (start 89.5 127.5) (end 90.5 128.5) (width 0.2) (layer "F.Cu") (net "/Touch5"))
 (segment (start 88.16 96.84) (end 70 115) (width 0.2) (layer "F.Cu") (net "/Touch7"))
 (segment (start 70 115) (end 63.75 115) (width 0.2) (layer "F.Cu") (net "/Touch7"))
 (segment (start 89.24 96.84) (end 88.16 96.84) (width 0.2) (layer "F.Cu") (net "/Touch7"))
 (segment (start 54.75 102.25) (end 54.75 154.5) (width 0.2) (layer "F.Cu") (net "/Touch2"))
 (segment (start 74 107) (end 72.946 105.946) (width 0.2) (layer "F.Cu") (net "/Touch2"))
 (segment (start 72.946 101.946) (end 72 101) (width 0.2) (layer "F.Cu") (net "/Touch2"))
 (segment (start 72.946 105.946) (end 72.946 101.946) (width 0.2) (layer "F.Cu") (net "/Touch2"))
 (segment (start 72 101) (end 56 101) (width 0.2) (layer "F.Cu") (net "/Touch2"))
 (segment (start 56 101) (end 54.75 102.25) (width 0.2) (layer "F.Cu") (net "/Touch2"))
 (segment (start 72.75 114) (end 72.75 154.5) (width 0.2) (layer "F.Cu") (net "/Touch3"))
 (segment (start 87.37 99.38) (end 72.75 114) (width 0.2) (layer "F.Cu") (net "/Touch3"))
 (segment (start 89.24 99.38) (end 87.37 99.38) (width 0.2) (layer "F.Cu") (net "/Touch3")))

